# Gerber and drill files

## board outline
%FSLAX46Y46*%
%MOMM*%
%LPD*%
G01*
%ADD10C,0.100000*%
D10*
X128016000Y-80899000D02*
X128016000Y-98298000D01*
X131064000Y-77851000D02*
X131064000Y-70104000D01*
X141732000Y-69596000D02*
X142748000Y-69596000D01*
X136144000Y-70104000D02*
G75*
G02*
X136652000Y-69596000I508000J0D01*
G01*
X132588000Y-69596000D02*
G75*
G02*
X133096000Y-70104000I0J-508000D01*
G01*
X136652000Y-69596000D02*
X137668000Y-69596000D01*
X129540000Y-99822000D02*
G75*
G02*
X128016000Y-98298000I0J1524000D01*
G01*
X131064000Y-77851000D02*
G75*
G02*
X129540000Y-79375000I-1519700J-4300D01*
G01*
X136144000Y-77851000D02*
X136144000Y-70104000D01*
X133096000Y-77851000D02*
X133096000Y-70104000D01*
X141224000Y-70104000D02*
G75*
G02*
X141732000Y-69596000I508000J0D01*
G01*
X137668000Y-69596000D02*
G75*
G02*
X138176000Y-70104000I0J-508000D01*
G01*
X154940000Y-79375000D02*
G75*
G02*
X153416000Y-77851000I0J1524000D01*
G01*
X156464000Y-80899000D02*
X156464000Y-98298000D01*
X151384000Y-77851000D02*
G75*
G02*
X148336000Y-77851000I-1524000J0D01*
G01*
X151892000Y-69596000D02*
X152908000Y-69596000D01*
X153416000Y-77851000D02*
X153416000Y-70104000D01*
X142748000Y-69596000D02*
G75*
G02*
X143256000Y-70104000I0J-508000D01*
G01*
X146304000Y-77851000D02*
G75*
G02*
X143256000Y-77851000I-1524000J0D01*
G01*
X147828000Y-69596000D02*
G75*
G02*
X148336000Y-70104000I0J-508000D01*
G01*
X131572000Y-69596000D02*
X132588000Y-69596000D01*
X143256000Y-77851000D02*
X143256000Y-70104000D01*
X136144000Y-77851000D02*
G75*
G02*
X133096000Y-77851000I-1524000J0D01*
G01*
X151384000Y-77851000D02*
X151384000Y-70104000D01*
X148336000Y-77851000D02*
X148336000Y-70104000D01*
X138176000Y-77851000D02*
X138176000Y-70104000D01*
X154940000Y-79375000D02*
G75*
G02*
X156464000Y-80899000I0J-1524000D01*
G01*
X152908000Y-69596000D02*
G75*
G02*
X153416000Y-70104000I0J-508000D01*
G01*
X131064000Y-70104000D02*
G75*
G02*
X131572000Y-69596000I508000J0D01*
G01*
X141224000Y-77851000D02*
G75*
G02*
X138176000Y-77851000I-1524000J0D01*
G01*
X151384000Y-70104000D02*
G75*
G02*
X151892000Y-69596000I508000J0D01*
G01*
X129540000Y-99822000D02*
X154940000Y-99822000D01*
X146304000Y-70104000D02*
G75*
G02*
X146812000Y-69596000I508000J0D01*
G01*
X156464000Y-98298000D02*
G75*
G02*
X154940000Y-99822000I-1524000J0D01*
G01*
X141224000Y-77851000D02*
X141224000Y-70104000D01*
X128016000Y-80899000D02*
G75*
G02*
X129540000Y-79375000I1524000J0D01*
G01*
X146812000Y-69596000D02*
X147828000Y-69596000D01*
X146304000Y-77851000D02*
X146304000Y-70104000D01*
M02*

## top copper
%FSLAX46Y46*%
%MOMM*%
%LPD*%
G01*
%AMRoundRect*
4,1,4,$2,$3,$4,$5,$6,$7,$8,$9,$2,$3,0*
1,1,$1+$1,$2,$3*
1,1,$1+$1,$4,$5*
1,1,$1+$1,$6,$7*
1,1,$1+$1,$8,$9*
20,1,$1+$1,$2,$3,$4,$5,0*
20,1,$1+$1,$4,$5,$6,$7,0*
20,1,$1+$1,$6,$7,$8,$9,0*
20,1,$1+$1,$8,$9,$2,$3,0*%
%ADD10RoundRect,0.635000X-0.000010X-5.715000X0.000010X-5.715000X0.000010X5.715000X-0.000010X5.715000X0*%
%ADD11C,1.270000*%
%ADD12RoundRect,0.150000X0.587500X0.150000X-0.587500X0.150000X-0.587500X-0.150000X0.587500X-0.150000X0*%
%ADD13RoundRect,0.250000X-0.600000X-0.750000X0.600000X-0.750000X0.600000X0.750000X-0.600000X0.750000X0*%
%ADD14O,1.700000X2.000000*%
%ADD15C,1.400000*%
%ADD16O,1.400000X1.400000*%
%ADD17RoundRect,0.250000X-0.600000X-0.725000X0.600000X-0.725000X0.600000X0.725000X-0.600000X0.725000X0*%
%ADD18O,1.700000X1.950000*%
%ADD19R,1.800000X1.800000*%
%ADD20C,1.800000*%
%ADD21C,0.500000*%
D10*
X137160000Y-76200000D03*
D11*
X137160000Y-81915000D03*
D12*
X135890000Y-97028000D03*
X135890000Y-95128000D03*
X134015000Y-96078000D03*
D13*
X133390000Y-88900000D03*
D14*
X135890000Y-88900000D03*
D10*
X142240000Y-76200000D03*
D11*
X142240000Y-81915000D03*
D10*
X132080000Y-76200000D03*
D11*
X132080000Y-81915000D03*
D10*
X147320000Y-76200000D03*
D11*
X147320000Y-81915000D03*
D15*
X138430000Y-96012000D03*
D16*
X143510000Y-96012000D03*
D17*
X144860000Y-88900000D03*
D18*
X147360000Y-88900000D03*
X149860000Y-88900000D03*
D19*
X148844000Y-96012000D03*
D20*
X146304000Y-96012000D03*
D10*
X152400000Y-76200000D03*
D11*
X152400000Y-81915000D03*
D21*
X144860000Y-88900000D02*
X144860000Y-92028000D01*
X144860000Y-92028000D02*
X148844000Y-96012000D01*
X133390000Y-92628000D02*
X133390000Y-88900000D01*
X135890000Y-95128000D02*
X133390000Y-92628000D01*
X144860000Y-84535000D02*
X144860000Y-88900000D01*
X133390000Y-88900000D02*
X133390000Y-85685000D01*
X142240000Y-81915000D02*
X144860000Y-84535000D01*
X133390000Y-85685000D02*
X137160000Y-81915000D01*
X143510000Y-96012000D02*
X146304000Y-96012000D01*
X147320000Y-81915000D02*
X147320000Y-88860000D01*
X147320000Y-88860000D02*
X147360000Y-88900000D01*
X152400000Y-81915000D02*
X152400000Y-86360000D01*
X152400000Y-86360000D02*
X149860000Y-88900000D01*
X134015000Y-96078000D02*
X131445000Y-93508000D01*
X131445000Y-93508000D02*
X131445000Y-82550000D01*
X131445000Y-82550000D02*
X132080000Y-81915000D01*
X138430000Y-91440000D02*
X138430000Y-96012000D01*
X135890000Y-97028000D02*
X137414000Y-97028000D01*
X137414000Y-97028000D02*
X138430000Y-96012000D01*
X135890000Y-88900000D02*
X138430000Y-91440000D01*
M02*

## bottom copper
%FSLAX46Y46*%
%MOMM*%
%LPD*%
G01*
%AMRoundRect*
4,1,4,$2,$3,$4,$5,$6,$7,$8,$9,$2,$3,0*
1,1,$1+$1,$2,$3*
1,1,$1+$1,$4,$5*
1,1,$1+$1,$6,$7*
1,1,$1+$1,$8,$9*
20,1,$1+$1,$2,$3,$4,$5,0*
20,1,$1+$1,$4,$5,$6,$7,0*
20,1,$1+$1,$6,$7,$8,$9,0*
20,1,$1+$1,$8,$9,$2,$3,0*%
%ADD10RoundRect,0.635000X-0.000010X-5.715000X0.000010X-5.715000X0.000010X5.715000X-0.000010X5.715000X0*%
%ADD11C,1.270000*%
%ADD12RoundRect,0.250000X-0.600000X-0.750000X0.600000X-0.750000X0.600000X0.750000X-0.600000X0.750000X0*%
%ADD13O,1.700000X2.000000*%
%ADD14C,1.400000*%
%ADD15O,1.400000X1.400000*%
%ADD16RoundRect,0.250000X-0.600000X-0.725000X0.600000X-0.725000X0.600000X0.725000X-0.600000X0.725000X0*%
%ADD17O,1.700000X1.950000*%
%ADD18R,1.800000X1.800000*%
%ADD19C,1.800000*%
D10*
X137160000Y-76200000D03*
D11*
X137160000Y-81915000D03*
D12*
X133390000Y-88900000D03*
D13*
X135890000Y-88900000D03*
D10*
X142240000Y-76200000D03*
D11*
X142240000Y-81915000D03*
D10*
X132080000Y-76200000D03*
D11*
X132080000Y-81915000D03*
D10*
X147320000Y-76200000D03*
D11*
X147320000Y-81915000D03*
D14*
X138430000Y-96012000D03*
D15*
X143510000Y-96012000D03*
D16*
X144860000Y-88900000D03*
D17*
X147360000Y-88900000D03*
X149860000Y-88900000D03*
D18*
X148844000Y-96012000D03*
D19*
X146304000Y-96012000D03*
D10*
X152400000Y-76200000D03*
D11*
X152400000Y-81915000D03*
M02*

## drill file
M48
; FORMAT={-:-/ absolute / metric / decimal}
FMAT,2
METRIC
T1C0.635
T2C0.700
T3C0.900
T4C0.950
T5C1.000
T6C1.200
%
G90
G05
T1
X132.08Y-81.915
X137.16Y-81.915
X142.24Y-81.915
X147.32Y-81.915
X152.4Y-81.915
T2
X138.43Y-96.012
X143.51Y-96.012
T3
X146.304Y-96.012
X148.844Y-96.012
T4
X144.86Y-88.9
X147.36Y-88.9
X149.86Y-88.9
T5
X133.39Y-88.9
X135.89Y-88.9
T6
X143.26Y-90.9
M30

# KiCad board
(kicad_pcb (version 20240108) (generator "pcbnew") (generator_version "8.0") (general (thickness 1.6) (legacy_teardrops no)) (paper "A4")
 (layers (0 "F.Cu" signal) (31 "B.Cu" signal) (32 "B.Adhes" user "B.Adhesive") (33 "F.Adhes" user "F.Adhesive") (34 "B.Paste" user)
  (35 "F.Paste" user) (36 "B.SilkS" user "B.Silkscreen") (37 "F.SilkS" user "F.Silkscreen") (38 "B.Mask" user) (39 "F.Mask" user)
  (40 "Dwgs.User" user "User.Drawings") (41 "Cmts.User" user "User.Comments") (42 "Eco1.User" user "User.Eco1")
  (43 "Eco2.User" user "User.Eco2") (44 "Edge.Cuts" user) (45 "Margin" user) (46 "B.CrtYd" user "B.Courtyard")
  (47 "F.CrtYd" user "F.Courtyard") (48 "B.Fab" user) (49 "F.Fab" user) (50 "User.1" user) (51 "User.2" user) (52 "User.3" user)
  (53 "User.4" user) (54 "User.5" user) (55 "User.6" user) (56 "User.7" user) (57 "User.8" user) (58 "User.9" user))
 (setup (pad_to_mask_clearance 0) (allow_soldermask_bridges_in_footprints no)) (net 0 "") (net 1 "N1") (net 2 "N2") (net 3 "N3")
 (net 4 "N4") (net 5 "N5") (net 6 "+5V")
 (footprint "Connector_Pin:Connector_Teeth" (layer "F.Cu") (at 137.16 76.2)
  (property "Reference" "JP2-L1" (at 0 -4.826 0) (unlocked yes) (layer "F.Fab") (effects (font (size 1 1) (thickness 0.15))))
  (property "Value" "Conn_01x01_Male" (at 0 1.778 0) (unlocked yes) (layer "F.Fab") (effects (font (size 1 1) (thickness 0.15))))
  (pad "1" smd roundrect (at 0 0) (size 1.27 12.7) (layers "F.Cu" "F.Paste" "F.Mask") (roundrect_rratio 0.5) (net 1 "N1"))
  (pad "1" smd roundrect (at 0 0) (size 1.27 12.7) (layers "B.Cu" "B.Paste" "B.Mask") (roundrect_rratio 0.5) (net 1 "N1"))
  (pad "1" thru_hole circle (at 0 5.715) (size 1.27 1.27) (drill 0.635) (layers "*.Cu" "*.Mask") (remove_unused_layers no) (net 1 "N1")))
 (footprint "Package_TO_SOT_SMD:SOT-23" (layer "F.Cu") (at 134.9525 96.078 180)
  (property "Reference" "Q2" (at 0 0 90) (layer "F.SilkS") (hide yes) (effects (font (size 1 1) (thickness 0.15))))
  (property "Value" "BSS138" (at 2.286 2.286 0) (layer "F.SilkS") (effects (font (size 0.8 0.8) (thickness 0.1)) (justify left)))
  (pad "1" smd roundrect (at -0.9375 -0.95 180) (size 1.475 0.6) (layers "F.Cu" "F.Paste" "F.Mask") (roundrect_rratio 0.25) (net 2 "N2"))
  (pad "2" smd roundrect (at -0.9375 0.95 180) (size 1.475 0.6) (layers "F.Cu" "F.Paste" "F.Mask") (roundrect_rratio 0.25) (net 1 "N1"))
  (pad "3" smd roundrect (at 0.9375 0 180) (size 1.475 0.6) (layers "F.Cu" "F.Paste" "F.Mask") (roundrect_rratio 0.25) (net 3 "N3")))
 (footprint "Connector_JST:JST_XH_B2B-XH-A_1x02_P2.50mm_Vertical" (layer "F.Cu") (at 133.39 88.9)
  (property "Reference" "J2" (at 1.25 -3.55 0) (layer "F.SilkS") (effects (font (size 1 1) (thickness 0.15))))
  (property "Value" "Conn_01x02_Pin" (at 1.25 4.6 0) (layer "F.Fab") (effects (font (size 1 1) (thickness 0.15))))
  (pad "1" thru_hole roundrect (at 0 0) (size 1.7 2) (drill 1) (layers "*.Cu" "*.Mask") (remove_unused_layers no)
   (roundrect_rratio 0.147059) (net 1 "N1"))
  (pad "2" thru_hole oval (at 2.5 0) (size 1.7 2) (drill 1) (layers "*.Cu" "*.Mask") (remove_unused_layers no) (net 2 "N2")))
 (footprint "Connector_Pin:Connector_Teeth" (layer "F.Cu") (at 142.24 76.2)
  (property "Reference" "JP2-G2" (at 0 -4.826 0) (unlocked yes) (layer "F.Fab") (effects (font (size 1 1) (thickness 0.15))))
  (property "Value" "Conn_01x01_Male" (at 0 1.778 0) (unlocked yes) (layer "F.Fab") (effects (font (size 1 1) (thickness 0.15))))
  (pad "1" smd roundrect (at 0 0) (size 1.27 12.7) (layers "F.Cu" "F.Paste" "F.Mask") (roundrect_rratio 0.5) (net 1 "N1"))
  (pad "1" smd roundrect (at 0 0) (size 1.27 12.7) (layers "B.Cu" "B.Paste" "B.Mask") (roundrect_rratio 0.5) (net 1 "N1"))
  (pad "1" thru_hole circle (at 0 5.715) (size 1.27 1.27) (drill 0.635) (layers "*.Cu" "*.Mask") (remove_unused_layers no) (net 1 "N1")))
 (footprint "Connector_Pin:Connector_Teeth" (layer "F.Cu") (at 132.08 76.2)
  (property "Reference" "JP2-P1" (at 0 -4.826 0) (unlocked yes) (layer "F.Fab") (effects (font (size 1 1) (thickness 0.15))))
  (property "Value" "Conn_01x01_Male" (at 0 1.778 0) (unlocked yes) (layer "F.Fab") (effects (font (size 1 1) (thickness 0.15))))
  (pad "1" smd roundrect (at 0 0) (size 1.27 12.7) (layers "F.Cu" "F.Paste" "F.Mask") (roundrect_rratio 0.5) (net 3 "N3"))
  (pad "1" smd roundrect (at 0 0) (size 1.27 12.7) (layers "B.Cu" "B.Paste" "B.Mask") (roundrect_rratio 0.5) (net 3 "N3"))
  (pad "1" thru_hole circle (at 0 5.715) (size 1.27 1.27) (drill 0.635) (layers "*.Cu" "*.Mask") (remove_unused_layers no) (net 3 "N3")))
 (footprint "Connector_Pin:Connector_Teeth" (layer "F.Cu") (at 147.32 76.2)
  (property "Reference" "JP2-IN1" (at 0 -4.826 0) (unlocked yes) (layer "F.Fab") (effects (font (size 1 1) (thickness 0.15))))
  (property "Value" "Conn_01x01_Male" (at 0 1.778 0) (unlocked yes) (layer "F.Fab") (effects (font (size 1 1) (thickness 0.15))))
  (pad "1" smd roundrect (at 0 0) (size 1.27 12.7) (layers "F.Cu" "F.Paste" "F.Mask") (roundrect_rratio 0.5) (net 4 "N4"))
  (pad "1" smd roundrect (at 0 0) (size 1.27 12.7) (layers "B.Cu" "B.Paste" "B.Mask") (roundrect_rratio 0.5) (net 4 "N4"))
  (pad "1" thru_hole circle (at 0 5.715) (size 1.27 1.27) (drill 0.635) (layers "*.Cu" "*.Mask") (remove_unused_layers no) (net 4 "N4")))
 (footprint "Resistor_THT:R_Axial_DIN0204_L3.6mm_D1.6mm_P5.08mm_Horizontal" (layer "F.Cu") (at 138.43 96.012)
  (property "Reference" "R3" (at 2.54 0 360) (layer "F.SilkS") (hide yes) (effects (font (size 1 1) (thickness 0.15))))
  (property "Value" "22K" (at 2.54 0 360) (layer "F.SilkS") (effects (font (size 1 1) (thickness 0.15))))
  (pad "1" thru_hole circle (at 0 0) (size 1.4 1.4) (drill 0.7) (layers "*.Cu" "*.Mask") (remove_unused_layers no) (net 2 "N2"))
  (pad "2" thru_hole oval (at 5.08 0) (size 1.4 1.4) (drill 0.7) (layers "*.Cu" "*.Mask") (remove_unused_layers no) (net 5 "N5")))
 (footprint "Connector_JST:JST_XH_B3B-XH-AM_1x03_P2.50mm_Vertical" (layer "F.Cu") (at 144.86 88.9)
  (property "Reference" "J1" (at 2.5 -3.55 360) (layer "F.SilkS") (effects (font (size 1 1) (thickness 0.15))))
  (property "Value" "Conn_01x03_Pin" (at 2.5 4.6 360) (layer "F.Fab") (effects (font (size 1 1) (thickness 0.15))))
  (pad "" np_thru_hole circle (at -1.6 2) (size 1.2 1.2) (drill 1.2) (layers "*.Cu" "*.Mask"))
  (pad "1" thru_hole roundrect (at 0 0) (size 1.7 1.95) (drill 0.95) (layers "*.Cu" "*.Mask") (remove_unused_layers no)
   (roundrect_rratio 0.147059) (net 1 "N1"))
  (pad "2" thru_hole oval (at 2.5 0) (size 1.7 1.95) (drill 0.95) (layers "*.Cu" "*.Mask") (remove_unused_layers no) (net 4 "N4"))
  (pad "3" thru_hole oval (at 5 0) (size 1.7 1.95) (drill 0.95) (layers "*.Cu" "*.Mask") (remove_unused_layers no) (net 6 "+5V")))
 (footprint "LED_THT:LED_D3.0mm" (layer "F.Cu") (at 148.844 96.012 180)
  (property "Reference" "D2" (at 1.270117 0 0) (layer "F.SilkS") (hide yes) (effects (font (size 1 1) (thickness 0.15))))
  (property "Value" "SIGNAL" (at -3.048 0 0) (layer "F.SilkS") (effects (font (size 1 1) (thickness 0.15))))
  (pad "1" thru_hole rect (at 0 0 180) (size 1.8 1.8) (drill 0.9) (layers "*.Cu" "*.Mask") (remove_unused_layers no) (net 1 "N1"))
  (pad "2" thru_hole circle (at 2.54 0 180) (size 1.8 1.8) (drill 0.9) (layers "*.Cu" "*.Mask") (remove_unused_layers no) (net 5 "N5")))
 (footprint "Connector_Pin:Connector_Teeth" (layer "F.Cu") (at 152.4 76.2)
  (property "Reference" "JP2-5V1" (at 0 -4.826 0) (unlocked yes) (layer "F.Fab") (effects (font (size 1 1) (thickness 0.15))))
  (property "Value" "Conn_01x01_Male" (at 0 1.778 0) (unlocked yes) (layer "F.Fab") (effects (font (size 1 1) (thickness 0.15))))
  (pad "1" smd roundrect (at 0 0) (size 1.27 12.7) (layers "F.Cu" "F.Paste" "F.Mask") (roundrect_rratio 0.5) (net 6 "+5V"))
  (pad "1" smd roundrect (at 0 0) (size 1.27 12.7) (layers "B.Cu" "B.Paste" "B.Mask") (roundrect_rratio 0.5) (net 6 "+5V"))
  (pad "1" thru_hole circle (at 0 5.715) (size 1.27 1.27) (drill 0.635) (layers "*.Cu" "*.Mask") (remove_unused_layers no) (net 6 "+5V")))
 (gr_line (start 128.016 80.899) (end 128.016 98.298) (stroke (width 0.1) (type solid)) (layer "Edge.Cuts"))
 (gr_line (start 131.064 77.851) (end 131.064 70.104) (stroke (width 0.1) (type solid)) (layer "Edge.Cuts"))
 (gr_line (start 141.732 69.596) (end 142.748 69.596) (stroke (width 0.1) (type solid)) (layer "Edge.Cuts"))
 (gr_arc (start 136.144 70.104) (mid 136.29279 69.74479) (end 136.652 69.596) (stroke (width 0.1) (type solid)) (layer "Edge.Cuts"))
 (gr_arc (start 132.588 69.596) (mid 132.94721 69.74479) (end 133.096 70.104) (stroke (width 0.1) (type solid)) (layer "Edge.Cuts"))
 (gr_line (start 136.652 69.596) (end 137.668 69.596) (stroke (width 0.1) (type solid)) (layer "Edge.Cuts"))
 (gr_arc (start 129.54 99.822) (mid 128.462369 99.375631) (end 128.016 98.298) (stroke (width 0.1) (type solid)) (layer "Edge.Cuts"))
 (gr_arc (start 131.064 77.851) (mid 130.618894 78.929894) (end 129.54 79.375) (stroke (width 0.1) (type solid)) (layer "Edge.Cuts"))
 (gr_line (start 136.144 77.851) (end 136.144 70.104) (stroke (width 0.1) (type solid)) (layer "Edge.Cuts"))
 (gr_line (start 133.096 77.851) (end 133.096 70.104) (stroke (width 0.1) (type solid)) (layer "Edge.Cuts"))
 (gr_arc (start 141.224 70.104) (mid 141.37279 69.74479) (end 141.732 69.596) (stroke (width 0.1) (type solid)) (layer "Edge.Cuts"))
 (gr_arc (start 137.668 69.596) (mid 138.02721 69.74479) (end 138.176 70.104) (stroke (width 0.1) (type solid)) (layer "Edge.Cuts"))
 (gr_arc (start 154.94 79.375) (mid 153.862369 78.928631) (end 153.416 77.851) (stroke (width 0.1) (type solid)) (layer "Edge.Cuts"))
 (gr_line (start 156.464 80.899) (end 156.464 98.298) (stroke (width 0.1) (type solid)) (layer "Edge.Cuts"))
 (gr_arc (start 151.384 77.851) (mid 149.86 79.375) (end 148.336 77.851) (stroke (width 0.1) (type solid)) (layer "Edge.Cuts"))
 (gr_line (start 151.892 69.596) (end 152.908 69.596) (stroke (width 0.1) (type solid)) (layer "Edge.Cuts"))
 (gr_line (start 153.416 77.851) (end 153.416 70.104) (stroke (width 0.1) (type solid)) (layer "Edge.Cuts"))
 (gr_arc (start 142.748 69.596) (mid 143.10721 69.74479) (end 143.256 70.104) (stroke (width 0.1) (type solid)) (layer "Edge.Cuts"))
 (gr_arc (start 146.304 77.851) (mid 144.78 79.375) (end 143.256 77.851) (stroke (width 0.1) (type solid)) (layer "Edge.Cuts"))
 (gr_arc (start 147.828 69.596) (mid 148.18721 69.74479) (end 148.336 70.104) (stroke (width 0.1) (type solid)) (layer "Edge.Cuts"))
 (gr_line (start 131.572 69.596) (end 132.588 69.596) (stroke (width 0.1) (type solid)) (layer "Edge.Cuts"))
 (gr_line (start 143.256 77.851) (end 143.256 70.104) (stroke (width 0.1) (type solid)) (layer "Edge.Cuts"))
 (gr_arc (start 136.144 77.851) (mid 134.62 79.375) (end 133.096 77.851) (stroke (width 0.1) (type solid)) (layer "Edge.Cuts"))
 (gr_line (start 151.384 77.851) (end 151.384 70.104) (stroke (width 0.1) (type solid)) (layer "Edge.Cuts"))
 (gr_line (start 148.336 77.851) (end 148.336 70.104) (stroke (width 0.1) (type solid)) (layer "Edge.Cuts"))
 (gr_line (start 138.176 77.851) (end 138.176 70.104) (stroke (width 0.1) (type solid)) (layer "Edge.Cuts"))
 (gr_arc (start 154.94 79.375) (mid 156.017631 79.821369) (end 156.464 80.899) (stroke (width 0.1) (type solid)) (layer "Edge.Cuts"))
 (gr_arc (start 152.908 69.596) (mid 153.26721 69.74479) (end 153.416 70.104) (stroke (width 0.1) (type solid)) (layer "Edge.Cuts"))
 (gr_arc (start 131.064 70.104) (mid 131.21279 69.74479) (end 131.572 69.596) (stroke (width 0.1) (type solid)) (layer "Edge.Cuts"))
 (gr_arc (start 141.224 77.851) (mid 139.7 79.375) (end 138.176 77.851) (stroke (width 0.1) (type solid)) (layer "Edge.Cuts"))
 (gr_arc (start 151.384 70.104) (mid 151.53279 69.74479) (end 151.892 69.596) (stroke (width 0.1) (type solid)) (layer "Edge.Cuts"))
 (gr_line (start 129.54 99.822) (end 154.94 99.822) (stroke (width 0.1) (type solid)) (layer "Edge.Cuts"))
 (gr_arc (start 146.304 70.104) (mid 146.45279 69.74479) (end 146.812 69.596) (stroke (width 0.1) (type solid)) (layer "Edge.Cuts"))
 (gr_arc (start 156.464 98.298) (mid 156.017631 99.375631) (end 154.94 99.822) (stroke (width 0.1) (type solid)) (layer "Edge.Cuts"))
 (gr_line (start 141.224 77.851) (end 141.224 70.104) (stroke (width 0.1) (type solid)) (layer "Edge.Cuts"))
 (gr_arc (start 128.016 80.899) (mid 128.462369 79.821369) (end 129.54 79.375) (stroke (width 0.1) (type solid)) (layer "Edge.Cuts"))
 (gr_line (start 146.812 69.596) (end 147.828 69.596) (stroke (width 0.1) (type solid)) (layer "Edge.Cuts"))
 (gr_line (start 146.304 77.851) (end 146.304 70.104) (stroke (width 0.1) (type solid)) (layer "Edge.Cuts"))
 (segment (start 144.86 88.9) (end 144.86 92.028) (width 0.5) (layer "F.Cu") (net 1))
 (segment (start 144.86 92.028) (end 148.844 96.012) (width 0.5) (layer "F.Cu") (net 1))
 (segment (start 133.39 92.628) (end 133.39 88.9) (width 0.5) (layer "F.Cu") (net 1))
 (segment (start 135.89 95.128) (end 133.39 92.628) (width 0.5) (layer "F.Cu") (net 1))
 (segment (start 144.86 84.535) (end 144.86 88.9) (width 0.5) (layer "F.Cu") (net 1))
 (segment (start 133.39 88.9) (end 133.39 85.685) (width 0.5) (layer "F.Cu") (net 1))
 (segment (start 142.24 81.915) (end 144.86 84.535) (width 0.5) (layer "F.Cu") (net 1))
 (segment (start 133.39 85.685) (end 137.16 81.915) (width 0.5) (layer "F.Cu") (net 1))
 (segment (start 143.51 96.012) (end 146.304 96.012) (width 0.5) (layer "F.Cu") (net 5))
 (segment (start 147.32 81.915) (end 147.32 88.86) (width 0.5) (layer "F.Cu") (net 4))
 (segment (start 147.32 88.86) (end 147.36 88.9) (width 0.5) (layer "F.Cu") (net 4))
 (segment (start 152.4 81.915) (end 152.4 86.36) (width 0.5) (layer "F.Cu") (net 6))
 (segment (start 152.4 86.36) (end 149.86 88.9) (width 0.5) (layer "F.Cu") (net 6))
 (segment (start 134.015 96.078) (end 131.445 93.508) (width 0.5) (layer "F.Cu") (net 3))
 (segment (start 131.445 93.508) (end 131.445 82.55) (width 0.5) (layer "F.Cu") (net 3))
 (segment (start 131.445 82.55) (end 132.08 81.915) (width 0.5) (layer "F.Cu") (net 3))
 (segment (start 138.43 91.44) (end 138.43 96.012) (width 0.5) (layer "F.Cu") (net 2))
 (segment (start 135.89 97.028) (end 137.414 97.028) (width 0.5) (layer "F.Cu") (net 2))
 (segment (start 137.414 97.028) (end 138.43 96.012) (width 0.5) (layer "F.Cu") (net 2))
 (segment (start 135.89 88.9) (end 138.43 91.44) (width 0.5) (layer "F.Cu") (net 2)))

